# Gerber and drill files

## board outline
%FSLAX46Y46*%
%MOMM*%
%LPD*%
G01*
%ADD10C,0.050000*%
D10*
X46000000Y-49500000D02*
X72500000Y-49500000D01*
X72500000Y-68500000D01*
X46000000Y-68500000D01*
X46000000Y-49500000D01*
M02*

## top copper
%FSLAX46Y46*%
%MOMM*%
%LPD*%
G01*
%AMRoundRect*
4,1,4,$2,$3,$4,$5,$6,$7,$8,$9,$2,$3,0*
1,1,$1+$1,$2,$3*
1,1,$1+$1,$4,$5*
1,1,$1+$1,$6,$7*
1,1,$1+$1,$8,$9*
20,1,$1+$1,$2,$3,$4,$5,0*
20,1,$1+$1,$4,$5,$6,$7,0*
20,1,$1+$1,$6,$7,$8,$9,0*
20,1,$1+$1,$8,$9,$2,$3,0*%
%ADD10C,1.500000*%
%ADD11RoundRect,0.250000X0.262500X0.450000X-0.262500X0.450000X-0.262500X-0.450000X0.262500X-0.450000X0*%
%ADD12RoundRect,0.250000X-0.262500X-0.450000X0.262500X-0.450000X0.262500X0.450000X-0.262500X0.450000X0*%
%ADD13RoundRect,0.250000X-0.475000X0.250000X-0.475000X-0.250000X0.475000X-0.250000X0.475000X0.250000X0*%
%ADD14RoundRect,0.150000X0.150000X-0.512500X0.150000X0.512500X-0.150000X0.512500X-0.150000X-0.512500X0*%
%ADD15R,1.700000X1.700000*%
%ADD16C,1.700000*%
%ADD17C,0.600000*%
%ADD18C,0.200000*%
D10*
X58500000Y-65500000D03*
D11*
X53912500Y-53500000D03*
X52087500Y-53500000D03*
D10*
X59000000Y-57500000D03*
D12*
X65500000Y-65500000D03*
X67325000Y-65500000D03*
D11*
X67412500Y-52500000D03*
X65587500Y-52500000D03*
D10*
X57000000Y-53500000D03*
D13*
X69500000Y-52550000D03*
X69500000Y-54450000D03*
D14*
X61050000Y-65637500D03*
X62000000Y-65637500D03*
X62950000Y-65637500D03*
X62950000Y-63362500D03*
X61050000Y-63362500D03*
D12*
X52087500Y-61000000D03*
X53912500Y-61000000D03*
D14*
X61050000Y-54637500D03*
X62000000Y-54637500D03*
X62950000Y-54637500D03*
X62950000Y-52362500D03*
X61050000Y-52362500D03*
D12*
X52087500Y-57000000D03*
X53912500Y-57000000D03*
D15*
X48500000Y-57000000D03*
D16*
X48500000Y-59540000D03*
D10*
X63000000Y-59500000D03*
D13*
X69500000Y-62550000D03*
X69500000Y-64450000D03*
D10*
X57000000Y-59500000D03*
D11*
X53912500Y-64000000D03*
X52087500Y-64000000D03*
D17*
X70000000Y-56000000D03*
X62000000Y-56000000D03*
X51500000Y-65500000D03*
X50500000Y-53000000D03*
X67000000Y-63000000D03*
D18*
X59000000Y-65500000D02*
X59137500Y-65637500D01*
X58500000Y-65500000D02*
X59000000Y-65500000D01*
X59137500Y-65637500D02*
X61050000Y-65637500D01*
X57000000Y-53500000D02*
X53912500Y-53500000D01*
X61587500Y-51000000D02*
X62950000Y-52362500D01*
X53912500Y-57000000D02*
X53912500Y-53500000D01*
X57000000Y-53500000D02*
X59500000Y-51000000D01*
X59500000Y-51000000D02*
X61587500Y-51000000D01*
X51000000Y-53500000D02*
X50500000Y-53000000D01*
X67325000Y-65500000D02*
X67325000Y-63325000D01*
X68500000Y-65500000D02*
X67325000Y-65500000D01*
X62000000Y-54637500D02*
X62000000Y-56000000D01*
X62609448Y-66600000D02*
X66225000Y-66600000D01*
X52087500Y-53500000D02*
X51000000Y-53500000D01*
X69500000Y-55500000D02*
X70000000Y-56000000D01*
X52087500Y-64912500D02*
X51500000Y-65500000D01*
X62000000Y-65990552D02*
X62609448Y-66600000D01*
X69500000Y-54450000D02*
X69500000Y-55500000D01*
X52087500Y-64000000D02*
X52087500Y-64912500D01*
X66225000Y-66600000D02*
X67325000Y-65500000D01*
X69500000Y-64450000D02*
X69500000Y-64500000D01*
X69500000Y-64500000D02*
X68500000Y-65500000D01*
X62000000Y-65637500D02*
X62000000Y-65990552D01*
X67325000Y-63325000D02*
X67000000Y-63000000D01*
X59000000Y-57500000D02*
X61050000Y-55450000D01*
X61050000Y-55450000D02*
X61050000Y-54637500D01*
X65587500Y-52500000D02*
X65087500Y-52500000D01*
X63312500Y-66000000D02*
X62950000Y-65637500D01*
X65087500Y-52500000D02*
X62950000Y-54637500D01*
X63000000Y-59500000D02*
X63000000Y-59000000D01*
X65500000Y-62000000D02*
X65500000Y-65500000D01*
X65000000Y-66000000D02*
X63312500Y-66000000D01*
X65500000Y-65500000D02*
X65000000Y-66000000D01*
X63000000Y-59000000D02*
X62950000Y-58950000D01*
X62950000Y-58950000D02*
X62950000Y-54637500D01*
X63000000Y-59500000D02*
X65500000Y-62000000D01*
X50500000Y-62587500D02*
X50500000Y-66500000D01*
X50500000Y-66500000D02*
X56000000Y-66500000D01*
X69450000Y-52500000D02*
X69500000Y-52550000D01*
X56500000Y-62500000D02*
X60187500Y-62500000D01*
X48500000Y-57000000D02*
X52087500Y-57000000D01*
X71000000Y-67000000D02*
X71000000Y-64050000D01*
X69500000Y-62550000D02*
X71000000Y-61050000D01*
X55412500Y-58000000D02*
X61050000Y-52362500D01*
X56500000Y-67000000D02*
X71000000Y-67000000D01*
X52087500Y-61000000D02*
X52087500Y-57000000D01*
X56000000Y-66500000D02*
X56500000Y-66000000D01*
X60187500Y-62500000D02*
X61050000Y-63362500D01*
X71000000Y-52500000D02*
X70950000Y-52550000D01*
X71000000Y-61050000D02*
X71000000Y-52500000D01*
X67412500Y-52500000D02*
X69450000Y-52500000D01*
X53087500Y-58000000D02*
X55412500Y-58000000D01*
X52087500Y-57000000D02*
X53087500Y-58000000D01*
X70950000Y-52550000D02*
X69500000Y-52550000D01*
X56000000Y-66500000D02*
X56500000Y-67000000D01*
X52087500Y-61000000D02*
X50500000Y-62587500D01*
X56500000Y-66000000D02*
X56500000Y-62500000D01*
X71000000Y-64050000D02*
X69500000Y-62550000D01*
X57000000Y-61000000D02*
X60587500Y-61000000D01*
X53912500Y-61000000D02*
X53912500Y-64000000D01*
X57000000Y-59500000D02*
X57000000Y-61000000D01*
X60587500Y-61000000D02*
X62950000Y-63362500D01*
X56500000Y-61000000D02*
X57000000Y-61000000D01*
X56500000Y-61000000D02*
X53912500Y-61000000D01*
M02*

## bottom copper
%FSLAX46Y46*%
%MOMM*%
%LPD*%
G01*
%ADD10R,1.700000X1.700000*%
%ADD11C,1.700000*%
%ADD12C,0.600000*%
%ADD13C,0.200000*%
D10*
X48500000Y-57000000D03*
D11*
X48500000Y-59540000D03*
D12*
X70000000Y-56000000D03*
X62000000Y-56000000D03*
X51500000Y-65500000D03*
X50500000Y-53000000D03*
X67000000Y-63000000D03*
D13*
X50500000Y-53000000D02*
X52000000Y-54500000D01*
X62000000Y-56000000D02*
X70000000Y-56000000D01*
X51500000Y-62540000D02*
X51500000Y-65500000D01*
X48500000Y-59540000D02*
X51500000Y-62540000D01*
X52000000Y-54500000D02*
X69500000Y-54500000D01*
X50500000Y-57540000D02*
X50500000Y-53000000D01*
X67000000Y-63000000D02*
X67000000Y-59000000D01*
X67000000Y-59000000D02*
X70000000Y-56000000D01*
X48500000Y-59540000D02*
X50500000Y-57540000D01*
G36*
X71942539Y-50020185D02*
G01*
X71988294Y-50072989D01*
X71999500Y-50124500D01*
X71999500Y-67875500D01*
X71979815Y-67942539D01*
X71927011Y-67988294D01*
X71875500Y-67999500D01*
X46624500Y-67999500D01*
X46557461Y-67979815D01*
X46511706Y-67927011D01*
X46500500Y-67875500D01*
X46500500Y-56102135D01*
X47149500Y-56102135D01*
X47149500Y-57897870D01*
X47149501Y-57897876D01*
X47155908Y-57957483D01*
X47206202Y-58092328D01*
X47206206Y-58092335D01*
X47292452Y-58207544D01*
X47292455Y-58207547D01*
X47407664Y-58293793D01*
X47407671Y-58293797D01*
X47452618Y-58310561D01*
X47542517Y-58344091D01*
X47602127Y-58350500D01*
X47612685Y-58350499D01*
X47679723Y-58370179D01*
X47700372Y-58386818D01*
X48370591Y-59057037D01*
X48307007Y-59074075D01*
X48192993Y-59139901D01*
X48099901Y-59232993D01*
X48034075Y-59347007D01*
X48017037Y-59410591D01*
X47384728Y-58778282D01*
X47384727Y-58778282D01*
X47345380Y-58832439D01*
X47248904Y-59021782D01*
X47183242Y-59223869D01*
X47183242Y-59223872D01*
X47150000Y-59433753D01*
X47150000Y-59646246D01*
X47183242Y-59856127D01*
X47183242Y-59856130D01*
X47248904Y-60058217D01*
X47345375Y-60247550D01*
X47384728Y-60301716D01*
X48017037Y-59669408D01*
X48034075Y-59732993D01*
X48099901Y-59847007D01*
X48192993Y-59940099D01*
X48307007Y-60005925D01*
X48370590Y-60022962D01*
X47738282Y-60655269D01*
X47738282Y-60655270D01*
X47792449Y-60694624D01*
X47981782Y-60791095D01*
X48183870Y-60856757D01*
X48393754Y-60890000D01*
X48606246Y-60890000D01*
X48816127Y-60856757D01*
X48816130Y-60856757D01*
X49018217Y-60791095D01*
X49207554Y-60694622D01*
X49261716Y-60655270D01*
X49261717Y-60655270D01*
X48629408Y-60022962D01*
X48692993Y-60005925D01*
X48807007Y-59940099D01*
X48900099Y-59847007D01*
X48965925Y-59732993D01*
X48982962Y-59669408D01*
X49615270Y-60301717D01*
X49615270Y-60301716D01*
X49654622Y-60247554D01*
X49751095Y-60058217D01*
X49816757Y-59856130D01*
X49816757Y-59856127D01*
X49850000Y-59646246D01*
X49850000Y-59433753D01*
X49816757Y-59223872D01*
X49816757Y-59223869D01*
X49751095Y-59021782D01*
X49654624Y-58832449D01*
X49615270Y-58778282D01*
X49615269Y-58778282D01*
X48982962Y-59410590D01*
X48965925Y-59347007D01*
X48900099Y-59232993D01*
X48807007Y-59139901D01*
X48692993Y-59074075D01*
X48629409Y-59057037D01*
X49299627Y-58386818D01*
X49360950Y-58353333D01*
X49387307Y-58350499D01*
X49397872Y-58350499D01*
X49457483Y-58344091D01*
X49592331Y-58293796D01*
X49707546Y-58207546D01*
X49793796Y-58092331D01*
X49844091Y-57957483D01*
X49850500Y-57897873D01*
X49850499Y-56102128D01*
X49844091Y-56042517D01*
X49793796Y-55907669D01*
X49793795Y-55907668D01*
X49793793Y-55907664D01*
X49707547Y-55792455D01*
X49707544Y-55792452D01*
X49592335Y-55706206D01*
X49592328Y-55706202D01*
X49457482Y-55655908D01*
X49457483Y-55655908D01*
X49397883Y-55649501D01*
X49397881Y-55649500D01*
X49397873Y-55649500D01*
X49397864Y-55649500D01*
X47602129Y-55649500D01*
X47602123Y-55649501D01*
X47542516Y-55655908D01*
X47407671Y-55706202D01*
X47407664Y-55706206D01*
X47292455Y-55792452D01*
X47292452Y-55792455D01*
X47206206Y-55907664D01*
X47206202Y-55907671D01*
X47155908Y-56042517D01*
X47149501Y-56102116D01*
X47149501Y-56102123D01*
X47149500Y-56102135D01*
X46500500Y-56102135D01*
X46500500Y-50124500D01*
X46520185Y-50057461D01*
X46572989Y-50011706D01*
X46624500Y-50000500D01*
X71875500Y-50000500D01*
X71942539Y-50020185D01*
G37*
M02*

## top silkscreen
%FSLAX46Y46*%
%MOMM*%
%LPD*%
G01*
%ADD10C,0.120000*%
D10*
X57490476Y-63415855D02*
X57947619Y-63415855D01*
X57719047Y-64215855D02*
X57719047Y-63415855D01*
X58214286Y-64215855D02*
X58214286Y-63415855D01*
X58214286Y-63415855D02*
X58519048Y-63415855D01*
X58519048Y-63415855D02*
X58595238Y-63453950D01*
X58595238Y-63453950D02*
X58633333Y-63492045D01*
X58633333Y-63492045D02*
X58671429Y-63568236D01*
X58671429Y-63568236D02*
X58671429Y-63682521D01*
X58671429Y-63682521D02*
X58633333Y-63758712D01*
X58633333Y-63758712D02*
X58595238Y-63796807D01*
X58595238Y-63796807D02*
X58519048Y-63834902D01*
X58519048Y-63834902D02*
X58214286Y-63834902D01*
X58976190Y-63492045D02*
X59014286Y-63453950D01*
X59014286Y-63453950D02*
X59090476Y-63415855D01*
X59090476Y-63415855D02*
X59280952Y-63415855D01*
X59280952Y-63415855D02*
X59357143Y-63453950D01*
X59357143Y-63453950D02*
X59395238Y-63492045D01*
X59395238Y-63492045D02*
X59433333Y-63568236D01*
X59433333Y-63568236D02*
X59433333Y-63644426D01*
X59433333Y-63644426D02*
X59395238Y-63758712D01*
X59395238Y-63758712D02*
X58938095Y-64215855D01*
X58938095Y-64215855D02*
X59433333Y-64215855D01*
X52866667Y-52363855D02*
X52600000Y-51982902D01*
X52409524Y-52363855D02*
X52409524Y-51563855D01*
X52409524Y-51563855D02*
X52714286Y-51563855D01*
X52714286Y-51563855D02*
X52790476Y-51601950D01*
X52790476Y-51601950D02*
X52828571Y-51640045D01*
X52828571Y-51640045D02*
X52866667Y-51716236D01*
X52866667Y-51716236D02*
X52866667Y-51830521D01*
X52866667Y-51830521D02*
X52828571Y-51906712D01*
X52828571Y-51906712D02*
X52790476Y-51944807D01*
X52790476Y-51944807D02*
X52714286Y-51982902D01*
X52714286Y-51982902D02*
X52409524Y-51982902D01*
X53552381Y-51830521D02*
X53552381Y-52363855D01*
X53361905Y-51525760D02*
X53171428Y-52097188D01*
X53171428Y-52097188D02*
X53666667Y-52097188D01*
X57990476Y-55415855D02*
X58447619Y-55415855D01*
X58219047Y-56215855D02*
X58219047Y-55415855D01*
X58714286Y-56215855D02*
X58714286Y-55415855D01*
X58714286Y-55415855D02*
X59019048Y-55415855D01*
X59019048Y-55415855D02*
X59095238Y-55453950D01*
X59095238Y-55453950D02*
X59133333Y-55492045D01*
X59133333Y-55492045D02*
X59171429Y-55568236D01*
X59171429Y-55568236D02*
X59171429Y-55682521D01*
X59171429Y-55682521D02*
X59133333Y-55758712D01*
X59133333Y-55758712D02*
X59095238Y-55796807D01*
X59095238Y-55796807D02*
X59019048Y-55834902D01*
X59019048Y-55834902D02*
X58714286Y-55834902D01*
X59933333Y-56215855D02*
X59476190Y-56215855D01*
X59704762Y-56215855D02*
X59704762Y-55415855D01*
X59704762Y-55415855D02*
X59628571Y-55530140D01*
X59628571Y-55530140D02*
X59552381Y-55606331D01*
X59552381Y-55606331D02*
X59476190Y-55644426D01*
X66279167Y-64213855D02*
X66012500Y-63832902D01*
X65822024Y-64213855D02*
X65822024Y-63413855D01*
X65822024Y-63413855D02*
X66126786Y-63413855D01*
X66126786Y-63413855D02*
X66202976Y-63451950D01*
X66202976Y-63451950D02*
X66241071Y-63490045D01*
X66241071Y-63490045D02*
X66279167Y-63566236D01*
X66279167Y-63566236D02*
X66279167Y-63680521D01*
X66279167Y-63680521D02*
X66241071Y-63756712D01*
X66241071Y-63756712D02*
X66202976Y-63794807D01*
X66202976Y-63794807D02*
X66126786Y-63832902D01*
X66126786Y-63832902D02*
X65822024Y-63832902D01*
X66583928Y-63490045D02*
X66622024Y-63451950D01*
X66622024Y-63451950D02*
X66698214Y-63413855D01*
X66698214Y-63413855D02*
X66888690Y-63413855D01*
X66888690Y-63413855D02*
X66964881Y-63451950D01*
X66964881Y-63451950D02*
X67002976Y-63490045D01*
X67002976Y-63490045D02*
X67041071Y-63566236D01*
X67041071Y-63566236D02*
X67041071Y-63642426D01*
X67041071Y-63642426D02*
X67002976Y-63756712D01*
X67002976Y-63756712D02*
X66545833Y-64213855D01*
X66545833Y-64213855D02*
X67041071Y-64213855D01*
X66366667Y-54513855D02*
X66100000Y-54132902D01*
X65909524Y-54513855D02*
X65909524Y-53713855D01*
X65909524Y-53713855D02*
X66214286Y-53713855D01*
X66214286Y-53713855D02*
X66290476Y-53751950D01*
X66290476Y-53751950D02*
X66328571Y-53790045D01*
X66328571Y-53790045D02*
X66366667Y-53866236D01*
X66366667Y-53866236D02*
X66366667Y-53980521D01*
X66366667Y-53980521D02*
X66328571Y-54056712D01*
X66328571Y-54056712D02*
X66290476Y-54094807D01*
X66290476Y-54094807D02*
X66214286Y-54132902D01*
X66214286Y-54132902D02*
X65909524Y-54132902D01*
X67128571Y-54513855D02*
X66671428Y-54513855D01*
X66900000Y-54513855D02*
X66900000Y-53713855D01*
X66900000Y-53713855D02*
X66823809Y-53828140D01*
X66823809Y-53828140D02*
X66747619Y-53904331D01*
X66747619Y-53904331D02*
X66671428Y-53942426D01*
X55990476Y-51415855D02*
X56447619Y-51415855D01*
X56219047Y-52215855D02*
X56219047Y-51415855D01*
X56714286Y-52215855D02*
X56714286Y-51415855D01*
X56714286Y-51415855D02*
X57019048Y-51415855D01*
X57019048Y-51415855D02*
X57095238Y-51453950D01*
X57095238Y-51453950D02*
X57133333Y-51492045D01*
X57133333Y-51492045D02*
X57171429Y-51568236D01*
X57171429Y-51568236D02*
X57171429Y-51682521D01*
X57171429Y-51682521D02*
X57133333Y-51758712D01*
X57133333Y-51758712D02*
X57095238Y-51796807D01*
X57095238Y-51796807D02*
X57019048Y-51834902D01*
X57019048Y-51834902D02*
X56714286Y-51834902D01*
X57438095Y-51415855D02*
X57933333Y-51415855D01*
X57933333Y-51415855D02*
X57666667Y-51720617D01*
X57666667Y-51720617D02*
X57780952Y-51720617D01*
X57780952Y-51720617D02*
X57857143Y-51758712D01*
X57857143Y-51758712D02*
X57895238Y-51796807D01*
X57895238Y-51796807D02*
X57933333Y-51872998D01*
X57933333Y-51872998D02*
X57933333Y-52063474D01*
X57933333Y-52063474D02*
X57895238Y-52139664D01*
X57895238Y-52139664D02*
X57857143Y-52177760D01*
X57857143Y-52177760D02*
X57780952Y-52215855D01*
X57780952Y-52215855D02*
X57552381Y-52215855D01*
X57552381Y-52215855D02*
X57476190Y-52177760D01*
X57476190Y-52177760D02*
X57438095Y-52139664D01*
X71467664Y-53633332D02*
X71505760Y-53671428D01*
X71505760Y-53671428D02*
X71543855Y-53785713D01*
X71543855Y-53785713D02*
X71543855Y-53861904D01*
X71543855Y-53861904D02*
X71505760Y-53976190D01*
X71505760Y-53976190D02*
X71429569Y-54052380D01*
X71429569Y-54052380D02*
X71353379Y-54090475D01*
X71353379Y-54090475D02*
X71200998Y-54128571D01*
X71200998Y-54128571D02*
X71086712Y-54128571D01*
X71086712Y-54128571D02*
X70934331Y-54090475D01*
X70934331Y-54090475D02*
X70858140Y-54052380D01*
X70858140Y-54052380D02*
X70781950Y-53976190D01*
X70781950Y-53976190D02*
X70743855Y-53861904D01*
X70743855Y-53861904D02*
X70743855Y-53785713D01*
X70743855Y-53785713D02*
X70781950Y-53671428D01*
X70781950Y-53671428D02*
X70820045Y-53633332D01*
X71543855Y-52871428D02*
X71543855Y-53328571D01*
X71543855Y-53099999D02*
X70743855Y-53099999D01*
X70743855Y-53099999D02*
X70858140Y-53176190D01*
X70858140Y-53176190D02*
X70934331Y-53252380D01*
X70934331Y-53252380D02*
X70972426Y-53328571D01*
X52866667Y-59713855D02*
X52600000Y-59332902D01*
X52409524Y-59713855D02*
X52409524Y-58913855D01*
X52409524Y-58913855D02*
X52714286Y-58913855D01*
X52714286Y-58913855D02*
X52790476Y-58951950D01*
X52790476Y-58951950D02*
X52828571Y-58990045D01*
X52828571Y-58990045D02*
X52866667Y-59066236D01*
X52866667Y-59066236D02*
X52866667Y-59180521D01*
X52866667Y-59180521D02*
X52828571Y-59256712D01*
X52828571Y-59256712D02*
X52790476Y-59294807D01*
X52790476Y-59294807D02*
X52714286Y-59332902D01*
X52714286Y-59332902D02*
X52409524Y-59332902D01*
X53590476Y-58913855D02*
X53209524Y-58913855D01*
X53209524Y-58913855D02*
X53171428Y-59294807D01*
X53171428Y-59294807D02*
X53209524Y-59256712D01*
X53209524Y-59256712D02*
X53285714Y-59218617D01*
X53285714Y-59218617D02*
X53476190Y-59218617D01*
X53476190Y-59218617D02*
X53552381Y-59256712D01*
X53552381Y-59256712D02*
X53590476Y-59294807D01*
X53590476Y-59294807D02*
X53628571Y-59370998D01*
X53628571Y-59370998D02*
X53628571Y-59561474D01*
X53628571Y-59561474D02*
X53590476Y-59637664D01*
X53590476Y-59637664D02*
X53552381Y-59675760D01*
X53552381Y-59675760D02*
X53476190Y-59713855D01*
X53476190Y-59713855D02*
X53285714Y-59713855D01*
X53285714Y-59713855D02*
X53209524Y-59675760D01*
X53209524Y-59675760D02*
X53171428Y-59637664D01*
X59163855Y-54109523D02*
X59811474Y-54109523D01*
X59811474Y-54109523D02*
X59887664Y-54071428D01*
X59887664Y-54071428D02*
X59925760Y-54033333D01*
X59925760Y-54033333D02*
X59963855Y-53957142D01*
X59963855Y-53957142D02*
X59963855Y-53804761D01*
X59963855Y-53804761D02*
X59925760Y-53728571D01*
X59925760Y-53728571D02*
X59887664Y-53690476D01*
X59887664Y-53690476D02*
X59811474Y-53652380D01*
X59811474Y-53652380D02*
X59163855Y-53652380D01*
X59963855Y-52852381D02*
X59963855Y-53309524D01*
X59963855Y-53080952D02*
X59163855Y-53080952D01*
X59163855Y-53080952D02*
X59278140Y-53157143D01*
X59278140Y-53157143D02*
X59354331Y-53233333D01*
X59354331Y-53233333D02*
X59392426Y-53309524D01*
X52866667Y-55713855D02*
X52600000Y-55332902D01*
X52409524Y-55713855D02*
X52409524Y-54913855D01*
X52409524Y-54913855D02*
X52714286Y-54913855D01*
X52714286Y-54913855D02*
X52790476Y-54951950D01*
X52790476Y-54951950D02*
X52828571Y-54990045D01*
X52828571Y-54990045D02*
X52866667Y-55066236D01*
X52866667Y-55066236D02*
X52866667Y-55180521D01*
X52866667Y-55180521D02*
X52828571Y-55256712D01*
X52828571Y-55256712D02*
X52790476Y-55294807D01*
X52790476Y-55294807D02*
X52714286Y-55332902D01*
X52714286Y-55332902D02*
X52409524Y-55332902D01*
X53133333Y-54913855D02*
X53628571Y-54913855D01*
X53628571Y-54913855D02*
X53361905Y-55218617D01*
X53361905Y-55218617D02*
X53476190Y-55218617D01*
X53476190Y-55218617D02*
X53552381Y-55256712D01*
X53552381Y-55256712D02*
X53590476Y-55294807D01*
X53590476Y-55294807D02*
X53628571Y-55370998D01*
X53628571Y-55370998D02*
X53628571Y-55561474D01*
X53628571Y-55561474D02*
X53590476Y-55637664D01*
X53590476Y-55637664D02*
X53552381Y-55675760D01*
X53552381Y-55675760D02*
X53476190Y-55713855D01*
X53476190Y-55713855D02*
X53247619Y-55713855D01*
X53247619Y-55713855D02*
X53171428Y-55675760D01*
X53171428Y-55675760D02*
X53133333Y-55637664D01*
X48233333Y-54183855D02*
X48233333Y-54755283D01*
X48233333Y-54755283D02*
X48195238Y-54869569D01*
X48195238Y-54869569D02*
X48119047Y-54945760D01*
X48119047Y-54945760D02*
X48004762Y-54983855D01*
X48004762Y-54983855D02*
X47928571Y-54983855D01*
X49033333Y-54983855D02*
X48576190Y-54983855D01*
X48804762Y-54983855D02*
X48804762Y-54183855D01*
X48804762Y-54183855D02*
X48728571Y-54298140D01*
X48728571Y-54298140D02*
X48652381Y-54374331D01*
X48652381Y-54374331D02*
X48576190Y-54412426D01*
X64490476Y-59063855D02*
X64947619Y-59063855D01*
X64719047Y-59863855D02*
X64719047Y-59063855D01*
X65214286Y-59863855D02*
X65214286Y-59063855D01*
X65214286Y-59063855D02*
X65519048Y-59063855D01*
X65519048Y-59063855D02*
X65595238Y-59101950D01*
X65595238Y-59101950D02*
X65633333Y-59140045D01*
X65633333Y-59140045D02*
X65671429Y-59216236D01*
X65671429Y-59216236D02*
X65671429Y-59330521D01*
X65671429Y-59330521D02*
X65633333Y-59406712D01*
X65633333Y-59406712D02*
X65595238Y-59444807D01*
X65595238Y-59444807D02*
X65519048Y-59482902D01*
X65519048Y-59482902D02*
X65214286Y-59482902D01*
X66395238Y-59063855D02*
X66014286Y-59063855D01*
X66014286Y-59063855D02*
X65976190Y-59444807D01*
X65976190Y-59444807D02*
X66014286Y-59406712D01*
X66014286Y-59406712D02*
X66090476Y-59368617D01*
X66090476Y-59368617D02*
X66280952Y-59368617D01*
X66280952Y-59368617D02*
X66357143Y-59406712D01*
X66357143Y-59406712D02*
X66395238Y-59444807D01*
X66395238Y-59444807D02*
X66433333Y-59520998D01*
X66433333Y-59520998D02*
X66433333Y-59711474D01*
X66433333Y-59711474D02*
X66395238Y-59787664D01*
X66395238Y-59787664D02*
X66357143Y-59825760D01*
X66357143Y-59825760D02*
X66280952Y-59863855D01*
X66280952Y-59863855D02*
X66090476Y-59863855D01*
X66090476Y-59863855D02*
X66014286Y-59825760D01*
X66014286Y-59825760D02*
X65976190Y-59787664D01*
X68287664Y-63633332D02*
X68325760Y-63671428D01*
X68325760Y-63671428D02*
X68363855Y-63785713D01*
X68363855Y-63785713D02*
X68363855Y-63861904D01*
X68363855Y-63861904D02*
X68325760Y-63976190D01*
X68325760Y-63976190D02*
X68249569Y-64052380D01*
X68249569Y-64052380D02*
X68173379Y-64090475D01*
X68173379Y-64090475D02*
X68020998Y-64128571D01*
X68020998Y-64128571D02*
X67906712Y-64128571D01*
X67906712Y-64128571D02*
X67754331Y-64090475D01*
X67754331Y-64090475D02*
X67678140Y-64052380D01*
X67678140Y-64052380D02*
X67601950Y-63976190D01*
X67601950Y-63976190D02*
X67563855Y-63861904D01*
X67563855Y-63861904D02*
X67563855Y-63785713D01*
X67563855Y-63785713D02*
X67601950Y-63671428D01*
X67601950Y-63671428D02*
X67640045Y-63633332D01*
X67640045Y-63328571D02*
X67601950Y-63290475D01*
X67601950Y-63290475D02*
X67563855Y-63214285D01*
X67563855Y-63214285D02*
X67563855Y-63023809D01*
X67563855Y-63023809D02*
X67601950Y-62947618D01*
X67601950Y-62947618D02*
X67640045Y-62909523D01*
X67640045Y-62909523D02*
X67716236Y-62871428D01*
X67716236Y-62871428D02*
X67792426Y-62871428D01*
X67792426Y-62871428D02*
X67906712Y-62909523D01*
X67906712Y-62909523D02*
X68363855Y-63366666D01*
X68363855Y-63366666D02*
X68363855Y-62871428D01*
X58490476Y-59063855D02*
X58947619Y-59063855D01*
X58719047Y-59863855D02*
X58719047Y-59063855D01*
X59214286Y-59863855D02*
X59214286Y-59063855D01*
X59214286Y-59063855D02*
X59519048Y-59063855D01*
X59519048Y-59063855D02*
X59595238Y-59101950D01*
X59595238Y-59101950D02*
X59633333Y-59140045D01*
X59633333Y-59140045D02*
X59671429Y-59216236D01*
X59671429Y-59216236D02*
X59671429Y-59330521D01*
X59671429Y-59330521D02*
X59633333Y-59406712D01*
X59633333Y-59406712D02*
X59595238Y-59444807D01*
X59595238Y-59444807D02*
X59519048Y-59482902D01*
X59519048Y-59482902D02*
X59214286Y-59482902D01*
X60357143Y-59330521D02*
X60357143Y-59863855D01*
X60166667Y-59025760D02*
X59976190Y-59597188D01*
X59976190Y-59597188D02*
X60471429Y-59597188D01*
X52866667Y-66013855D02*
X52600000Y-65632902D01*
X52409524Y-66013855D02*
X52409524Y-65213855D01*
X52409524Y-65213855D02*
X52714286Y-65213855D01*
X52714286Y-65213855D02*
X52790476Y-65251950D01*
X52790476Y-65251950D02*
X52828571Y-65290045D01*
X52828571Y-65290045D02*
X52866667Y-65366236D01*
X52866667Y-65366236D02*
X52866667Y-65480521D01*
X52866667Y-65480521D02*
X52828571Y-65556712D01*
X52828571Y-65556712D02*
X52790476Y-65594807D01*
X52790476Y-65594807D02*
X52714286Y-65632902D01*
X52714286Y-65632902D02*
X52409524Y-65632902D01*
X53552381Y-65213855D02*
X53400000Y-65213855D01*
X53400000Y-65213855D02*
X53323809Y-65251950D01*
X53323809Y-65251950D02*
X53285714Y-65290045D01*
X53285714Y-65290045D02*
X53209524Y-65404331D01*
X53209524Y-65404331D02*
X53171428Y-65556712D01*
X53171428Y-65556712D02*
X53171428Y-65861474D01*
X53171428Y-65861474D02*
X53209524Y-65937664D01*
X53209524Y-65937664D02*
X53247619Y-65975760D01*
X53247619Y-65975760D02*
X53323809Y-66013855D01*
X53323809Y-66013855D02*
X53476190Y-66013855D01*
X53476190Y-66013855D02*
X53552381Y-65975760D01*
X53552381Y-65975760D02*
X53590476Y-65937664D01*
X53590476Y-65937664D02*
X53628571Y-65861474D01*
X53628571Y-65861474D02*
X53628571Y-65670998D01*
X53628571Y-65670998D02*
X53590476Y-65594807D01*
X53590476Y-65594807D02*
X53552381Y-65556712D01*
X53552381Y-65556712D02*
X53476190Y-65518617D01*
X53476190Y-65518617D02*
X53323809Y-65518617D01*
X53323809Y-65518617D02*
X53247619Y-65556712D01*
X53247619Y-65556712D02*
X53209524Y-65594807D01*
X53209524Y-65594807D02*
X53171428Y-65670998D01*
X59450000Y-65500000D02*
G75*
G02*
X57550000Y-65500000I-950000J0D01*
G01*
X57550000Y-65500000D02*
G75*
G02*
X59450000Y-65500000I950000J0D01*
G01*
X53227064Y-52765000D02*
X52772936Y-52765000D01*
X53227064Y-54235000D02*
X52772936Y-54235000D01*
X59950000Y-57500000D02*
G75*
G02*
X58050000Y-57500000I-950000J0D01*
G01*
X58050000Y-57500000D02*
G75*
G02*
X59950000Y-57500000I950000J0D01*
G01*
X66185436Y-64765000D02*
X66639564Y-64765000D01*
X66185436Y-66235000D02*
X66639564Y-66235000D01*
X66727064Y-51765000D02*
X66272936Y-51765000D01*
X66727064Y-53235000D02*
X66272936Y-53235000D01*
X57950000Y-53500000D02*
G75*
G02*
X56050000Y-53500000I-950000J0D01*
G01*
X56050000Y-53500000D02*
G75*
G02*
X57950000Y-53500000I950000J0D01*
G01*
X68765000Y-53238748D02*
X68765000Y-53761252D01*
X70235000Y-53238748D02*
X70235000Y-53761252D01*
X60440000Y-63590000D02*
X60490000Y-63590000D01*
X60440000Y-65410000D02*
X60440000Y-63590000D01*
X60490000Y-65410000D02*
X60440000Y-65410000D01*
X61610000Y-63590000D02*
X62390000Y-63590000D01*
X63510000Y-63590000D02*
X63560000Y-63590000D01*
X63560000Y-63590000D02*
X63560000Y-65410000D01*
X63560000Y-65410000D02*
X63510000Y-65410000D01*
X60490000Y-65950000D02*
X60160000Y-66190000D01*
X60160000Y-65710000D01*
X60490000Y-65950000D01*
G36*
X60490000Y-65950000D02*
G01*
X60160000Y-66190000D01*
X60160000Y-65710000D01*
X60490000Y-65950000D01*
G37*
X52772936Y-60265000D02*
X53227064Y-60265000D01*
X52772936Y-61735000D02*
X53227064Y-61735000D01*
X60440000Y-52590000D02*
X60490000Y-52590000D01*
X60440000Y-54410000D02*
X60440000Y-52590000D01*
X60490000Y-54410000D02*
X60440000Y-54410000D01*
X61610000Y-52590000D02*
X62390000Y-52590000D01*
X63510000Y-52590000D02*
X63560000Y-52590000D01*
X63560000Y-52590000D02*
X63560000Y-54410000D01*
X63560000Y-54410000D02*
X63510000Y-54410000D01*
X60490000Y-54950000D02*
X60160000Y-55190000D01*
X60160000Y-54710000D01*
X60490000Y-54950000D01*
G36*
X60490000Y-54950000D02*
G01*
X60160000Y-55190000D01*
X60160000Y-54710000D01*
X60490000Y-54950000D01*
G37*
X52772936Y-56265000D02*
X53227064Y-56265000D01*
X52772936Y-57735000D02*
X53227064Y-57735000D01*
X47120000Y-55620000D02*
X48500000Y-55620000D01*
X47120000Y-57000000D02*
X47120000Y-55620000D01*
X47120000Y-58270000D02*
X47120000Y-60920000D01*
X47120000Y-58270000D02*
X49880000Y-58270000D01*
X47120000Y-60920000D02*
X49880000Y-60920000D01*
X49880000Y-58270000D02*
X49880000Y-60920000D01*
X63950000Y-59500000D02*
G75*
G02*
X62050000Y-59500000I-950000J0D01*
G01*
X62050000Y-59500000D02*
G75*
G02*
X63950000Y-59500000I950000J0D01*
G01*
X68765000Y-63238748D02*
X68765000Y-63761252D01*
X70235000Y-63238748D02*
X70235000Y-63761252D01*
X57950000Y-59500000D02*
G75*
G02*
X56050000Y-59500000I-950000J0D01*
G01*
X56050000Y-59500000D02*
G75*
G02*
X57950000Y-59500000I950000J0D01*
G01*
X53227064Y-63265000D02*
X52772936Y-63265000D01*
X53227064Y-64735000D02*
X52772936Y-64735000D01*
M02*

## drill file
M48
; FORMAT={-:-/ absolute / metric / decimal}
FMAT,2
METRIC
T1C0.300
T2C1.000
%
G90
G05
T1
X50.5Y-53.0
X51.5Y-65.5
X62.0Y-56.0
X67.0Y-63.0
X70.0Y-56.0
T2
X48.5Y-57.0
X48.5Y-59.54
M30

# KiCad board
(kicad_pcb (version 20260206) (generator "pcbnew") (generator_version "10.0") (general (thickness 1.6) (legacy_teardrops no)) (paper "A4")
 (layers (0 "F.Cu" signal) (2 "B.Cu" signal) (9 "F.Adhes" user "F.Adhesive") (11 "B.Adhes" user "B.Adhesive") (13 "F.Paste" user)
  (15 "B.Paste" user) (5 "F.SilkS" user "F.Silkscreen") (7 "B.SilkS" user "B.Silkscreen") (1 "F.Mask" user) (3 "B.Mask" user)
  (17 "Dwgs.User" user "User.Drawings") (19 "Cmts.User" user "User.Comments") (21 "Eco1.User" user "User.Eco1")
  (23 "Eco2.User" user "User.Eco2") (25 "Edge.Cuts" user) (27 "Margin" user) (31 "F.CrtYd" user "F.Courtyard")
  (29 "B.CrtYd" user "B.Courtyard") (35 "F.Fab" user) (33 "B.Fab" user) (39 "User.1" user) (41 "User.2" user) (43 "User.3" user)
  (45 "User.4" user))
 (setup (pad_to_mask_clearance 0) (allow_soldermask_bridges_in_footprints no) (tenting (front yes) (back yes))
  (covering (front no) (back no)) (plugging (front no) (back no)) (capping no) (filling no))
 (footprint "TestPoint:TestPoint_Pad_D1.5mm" (layer "F.Cu") (at 58.5 65.5)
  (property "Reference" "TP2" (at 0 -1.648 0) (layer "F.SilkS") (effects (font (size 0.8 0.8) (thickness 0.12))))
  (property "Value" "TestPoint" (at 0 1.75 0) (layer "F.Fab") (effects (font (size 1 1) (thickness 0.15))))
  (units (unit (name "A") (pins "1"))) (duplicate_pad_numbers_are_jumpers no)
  (fp_circle (center 0 0) (end 0 0.95) (stroke (width 0.12) (type solid)) (fill no) (layer "F.SilkS"))
  (pad "1" smd circle (at 0 0) (size 1.5 1.5) (layers "F.Cu" "F.Mask") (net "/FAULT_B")))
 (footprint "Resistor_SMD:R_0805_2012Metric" (layer "F.Cu") (at 53 53.5 180)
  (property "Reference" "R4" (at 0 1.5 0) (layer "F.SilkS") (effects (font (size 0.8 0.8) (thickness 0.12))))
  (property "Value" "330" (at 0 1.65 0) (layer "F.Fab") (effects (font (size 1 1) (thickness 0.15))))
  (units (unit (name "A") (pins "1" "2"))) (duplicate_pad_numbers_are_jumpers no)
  (fp_line (start -0.227064 0.735) (end 0.227064 0.735) (stroke (width 0.12) (type solid)) (layer "F.SilkS"))
  (fp_line (start -0.227064 -0.735) (end 0.227064 -0.735) (stroke (width 0.12) (type solid)) (layer "F.SilkS"))
  (pad "1" smd roundrect (at -0.9125 0 180) (size 1.025 1.4) (layers "F.Cu" "F.Mask" "F.Paste") (roundrect_rratio 0.243902) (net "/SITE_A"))
  (pad "2" smd roundrect (at 0.9125 0 180) (size 1.025 1.4) (layers "F.Cu" "F.Mask" "F.Paste") (roundrect_rratio 0.243902) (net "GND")))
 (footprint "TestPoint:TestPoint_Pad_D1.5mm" (layer "F.Cu") (at 59 57.5)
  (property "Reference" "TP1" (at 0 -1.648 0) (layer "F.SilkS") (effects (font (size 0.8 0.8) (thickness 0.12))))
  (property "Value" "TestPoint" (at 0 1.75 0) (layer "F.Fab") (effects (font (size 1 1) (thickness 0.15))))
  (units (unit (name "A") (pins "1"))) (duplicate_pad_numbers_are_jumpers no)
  (fp_circle (center 0 0) (end 0 0.95) (stroke (width 0.12) (type solid)) (fill no) (layer "F.SilkS"))
  (pad "1" smd circle (at 0 0) (size 1.5 1.5) (layers "F.Cu" "F.Mask") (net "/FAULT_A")))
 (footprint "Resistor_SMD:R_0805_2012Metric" (layer "F.Cu") (at 66.4125 65.5)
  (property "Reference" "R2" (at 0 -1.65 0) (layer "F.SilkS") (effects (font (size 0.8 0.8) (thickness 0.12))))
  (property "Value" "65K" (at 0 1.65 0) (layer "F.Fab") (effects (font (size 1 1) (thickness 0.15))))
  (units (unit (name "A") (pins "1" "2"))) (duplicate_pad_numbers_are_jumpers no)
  (fp_line (start -0.227064 -0.735) (end 0.227064 -0.735) (stroke (width 0.12) (type solid)) (layer "F.SilkS"))
  (fp_line (start -0.227064 0.735) (end 0.227064 0.735) (stroke (width 0.12) (type solid)) (layer "F.SilkS"))
  (pad "1" smd roundrect (at -0.9125 0) (size 1.025 1.4) (layers "F.Cu" "F.Mask" "F.Paste") (roundrect_rratio 0.243902) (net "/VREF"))
  (pad "2" smd roundrect (at 0.9125 0) (size 1.025 1.4) (layers "F.Cu" "F.Mask" "F.Paste") (roundrect_rratio 0.243902) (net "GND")))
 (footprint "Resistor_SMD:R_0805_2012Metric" (layer "F.Cu") (at 66.5 52.5 180)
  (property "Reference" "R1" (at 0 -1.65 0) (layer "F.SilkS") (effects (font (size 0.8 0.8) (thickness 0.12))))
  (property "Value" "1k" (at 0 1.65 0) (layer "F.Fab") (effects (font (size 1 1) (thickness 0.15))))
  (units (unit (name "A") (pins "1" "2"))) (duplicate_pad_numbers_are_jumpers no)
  (fp_line (start -0.227064 0.735) (end 0.227064 0.735) (stroke (width 0.12) (type solid)) (layer "F.SilkS"))
  (fp_line (start -0.227064 -0.735) (end 0.227064 -0.735) (stroke (width 0.12) (type solid)) (layer "F.SilkS"))
  (pad "1" smd roundrect (at -0.9125 0 180) (size 1.025 1.4) (layers "F.Cu" "F.Mask" "F.Paste") (roundrect_rratio 0.243902) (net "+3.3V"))
  (pad "2" smd roundrect (at 0.9125 0 180) (size 1.025 1.4) (layers "F.Cu" "F.Mask" "F.Paste") (roundrect_rratio 0.243902) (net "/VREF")))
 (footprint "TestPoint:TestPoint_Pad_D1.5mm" (layer "F.Cu") (at 57 53.5)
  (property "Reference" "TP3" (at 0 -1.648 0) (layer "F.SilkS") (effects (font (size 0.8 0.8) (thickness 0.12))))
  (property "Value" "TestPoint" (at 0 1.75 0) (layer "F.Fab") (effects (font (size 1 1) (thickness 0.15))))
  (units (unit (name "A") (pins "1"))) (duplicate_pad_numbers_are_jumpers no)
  (fp_circle (center 0 0) (end 0 0.95) (stroke (width 0.12) (type solid)) (fill no) (layer "F.SilkS"))
  (pad "1" smd circle (at 0 0) (size 1.5 1.5) (layers "F.Cu" "F.Mask") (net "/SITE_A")))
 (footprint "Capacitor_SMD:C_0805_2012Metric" (layer "F.Cu") (at 69.5 53.5 -90)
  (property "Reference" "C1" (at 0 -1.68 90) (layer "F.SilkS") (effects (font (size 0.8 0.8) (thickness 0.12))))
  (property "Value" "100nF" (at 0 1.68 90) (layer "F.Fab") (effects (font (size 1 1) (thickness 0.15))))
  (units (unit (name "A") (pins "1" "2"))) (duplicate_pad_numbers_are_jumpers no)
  (fp_line (start -0.261252 0.735) (end 0.261252 0.735) (stroke (width 0.12) (type solid)) (layer "F.SilkS"))
  (fp_line (start -0.261252 -0.735) (end 0.261252 -0.735) (stroke (width 0.12) (type solid)) (layer "F.SilkS"))
  (pad "1" smd roundrect (at -0.95 0 270) (size 1 1.45) (layers "F.Cu" "F.Mask" "F.Paste") (roundrect_rratio 0.25) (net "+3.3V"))
  (pad "2" smd roundrect (at 0.95 0 270) (size 1 1.45) (layers "F.Cu" "F.Mask" "F.Paste") (roundrect_rratio 0.25) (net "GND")))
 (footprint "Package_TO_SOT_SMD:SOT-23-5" (layer "F.Cu") (at 62 64.5 90)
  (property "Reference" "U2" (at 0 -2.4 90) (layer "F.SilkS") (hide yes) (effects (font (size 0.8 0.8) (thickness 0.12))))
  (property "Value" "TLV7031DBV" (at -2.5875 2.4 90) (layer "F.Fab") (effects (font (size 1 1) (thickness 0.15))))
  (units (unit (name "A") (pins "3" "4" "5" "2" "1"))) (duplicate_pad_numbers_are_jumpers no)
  (fp_line (start 0.91 -1.56) (end 0.91 -1.51) (stroke (width 0.12) (type solid)) (layer "F.SilkS"))
  (fp_line (start -0.91 -1.56) (end 0.91 -1.56) (stroke (width 0.12) (type solid)) (layer "F.SilkS"))
  (fp_line (start -0.91 -1.51) (end -0.91 -1.56) (stroke (width 0.12) (type solid)) (layer "F.SilkS"))
  (fp_line (start 0.91 -0.39) (end 0.91 0.39) (stroke (width 0.12) (type solid)) (layer "F.SilkS"))
  (fp_line (start 0.91 1.51) (end 0.91 1.56) (stroke (width 0.12) (type solid)) (layer "F.SilkS"))
  (fp_line (start 0.91 1.56) (end -0.91 1.56) (stroke (width 0.12) (type solid)) (layer "F.SilkS"))
  (fp_line (start -0.91 1.56) (end -0.91 1.51) (stroke (width 0.12) (type solid)) (layer "F.SilkS"))
  (fp_poly (pts (xy -1.45 -1.51) (xy -1.69 -1.84) (xy -1.21 -1.84)) (stroke (width 0.12) (type solid)) (fill yes) (layer "F.SilkS"))
  (pad "1" smd roundrect (at -1.1375 -0.95 90) (size 1.325 0.6) (layers "F.Cu" "F.Mask" "F.Paste") (roundrect_rratio 0.25) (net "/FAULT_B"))
  (pad "2" smd roundrect (at -1.1375 0 90) (size 1.325 0.6) (layers "F.Cu" "F.Mask" "F.Paste") (roundrect_rratio 0.25) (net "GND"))
  (pad "3" smd roundrect (at -1.1375 0.95 90) (size 1.325 0.6) (layers "F.Cu" "F.Mask" "F.Paste") (roundrect_rratio 0.25) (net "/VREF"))
  (pad "4" smd roundrect (at 1.1375 0.95 90) (size 1.325 0.6) (layers "F.Cu" "F.Mask" "F.Paste") (roundrect_rratio 0.25) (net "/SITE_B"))
  (pad "5" smd roundrect (at 1.1375 -0.95 90) (size 1.325 0.6) (layers "F.Cu" "F.Mask" "F.Paste") (roundrect_rratio 0.25) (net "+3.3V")))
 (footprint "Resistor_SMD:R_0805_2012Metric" (layer "F.Cu") (at 53 61)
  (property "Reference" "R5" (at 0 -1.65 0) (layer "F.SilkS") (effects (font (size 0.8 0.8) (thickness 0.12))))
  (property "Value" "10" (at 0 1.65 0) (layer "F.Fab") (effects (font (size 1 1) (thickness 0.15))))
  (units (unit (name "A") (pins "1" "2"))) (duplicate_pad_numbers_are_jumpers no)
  (fp_line (start -0.227064 -0.735) (end 0.227064 -0.735) (stroke (width 0.12) (type solid)) (layer "F.SilkS"))
  (fp_line (start -0.227064 0.735) (end 0.227064 0.735) (stroke (width 0.12) (type solid)) (layer "F.SilkS"))
  (pad "1" smd roundrect (at -0.9125 0) (size 1.025 1.4) (layers "F.Cu" "F.Mask" "F.Paste") (roundrect_rratio 0.243902) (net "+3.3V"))
  (pad "2" smd roundrect (at 0.9125 0) (size 1.025 1.4) (layers "F.Cu" "F.Mask" "F.Paste") (roundrect_rratio 0.243902) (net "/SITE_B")))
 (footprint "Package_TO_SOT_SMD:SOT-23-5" (layer "F.Cu") (at 62 53.5 90)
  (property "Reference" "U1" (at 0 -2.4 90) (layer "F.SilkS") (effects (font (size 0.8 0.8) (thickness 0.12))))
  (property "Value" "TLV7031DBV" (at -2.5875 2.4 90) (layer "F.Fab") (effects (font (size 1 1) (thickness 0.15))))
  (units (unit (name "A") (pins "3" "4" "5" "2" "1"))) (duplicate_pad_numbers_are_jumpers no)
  (fp_line (start 0.91 -1.56) (end 0.91 -1.51) (stroke (width 0.12) (type solid)) (layer "F.SilkS"))
  (fp_line (start -0.91 -1.56) (end 0.91 -1.56) (stroke (width 0.12) (type solid)) (layer "F.SilkS"))
  (fp_line (start -0.91 -1.51) (end -0.91 -1.56) (stroke (width 0.12) (type solid)) (layer "F.SilkS"))
  (fp_line (start 0.91 -0.39) (end 0.91 0.39) (stroke (width 0.12) (type solid)) (layer "F.SilkS"))
  (fp_line (start 0.91 1.51) (end 0.91 1.56) (stroke (width 0.12) (type solid)) (layer "F.SilkS"))
  (fp_line (start 0.91 1.56) (end -0.91 1.56) (stroke (width 0.12) (type solid)) (layer "F.SilkS"))
  (fp_line (start -0.91 1.56) (end -0.91 1.51) (stroke (width 0.12) (type solid)) (layer "F.SilkS"))
  (fp_poly (pts (xy -1.45 -1.51) (xy -1.69 -1.84) (xy -1.21 -1.84)) (stroke (width 0.12) (type solid)) (fill yes) (layer "F.SilkS"))
  (pad "1" smd roundrect (at -1.1375 -0.95 90) (size 1.325 0.6) (layers "F.Cu" "F.Mask" "F.Paste") (roundrect_rratio 0.25) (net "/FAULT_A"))
  (pad "2" smd roundrect (at -1.1375 0 90) (size 1.325 0.6) (layers "F.Cu" "F.Mask" "F.Paste") (roundrect_rratio 0.25) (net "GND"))
  (pad "3" smd roundrect (at -1.1375 0.95 90) (size 1.325 0.6) (layers "F.Cu" "F.Mask" "F.Paste") (roundrect_rratio 0.25) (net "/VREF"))
  (pad "4" smd roundrect (at 1.1375 0.95 90) (size 1.325 0.6) (layers "F.Cu" "F.Mask" "F.Paste") (roundrect_rratio 0.25) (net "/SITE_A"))
  (pad "5" smd roundrect (at 1.1375 -0.95 90) (size 1.325 0.6) (layers "F.Cu" "F.Mask" "F.Paste") (roundrect_rratio 0.25) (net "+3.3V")))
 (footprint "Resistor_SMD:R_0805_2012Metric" (layer "F.Cu") (at 53 57)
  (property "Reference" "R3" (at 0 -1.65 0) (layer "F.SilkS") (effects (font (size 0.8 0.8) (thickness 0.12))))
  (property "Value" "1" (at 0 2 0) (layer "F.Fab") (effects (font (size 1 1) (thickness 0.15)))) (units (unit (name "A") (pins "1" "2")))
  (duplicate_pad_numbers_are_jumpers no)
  (fp_line (start -0.227064 -0.735) (end 0.227064 -0.735) (stroke (width 0.12) (type solid)) (layer "F.SilkS"))
  (fp_line (start -0.227064 0.735) (end 0.227064 0.735) (stroke (width 0.12) (type solid)) (layer "F.SilkS"))
  (pad "1" smd roundrect (at -0.9125 0) (size 1.025 1.4) (layers "F.Cu" "F.Mask" "F.Paste") (roundrect_rratio 0.243902) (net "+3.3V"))
  (pad "2" smd roundrect (at 0.9125 0) (size 1.025 1.4) (layers "F.Cu" "F.Mask" "F.Paste") (roundrect_rratio 0.243902) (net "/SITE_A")))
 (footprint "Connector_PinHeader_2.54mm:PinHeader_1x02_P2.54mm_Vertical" (layer "F.Cu") (at 48.5 57)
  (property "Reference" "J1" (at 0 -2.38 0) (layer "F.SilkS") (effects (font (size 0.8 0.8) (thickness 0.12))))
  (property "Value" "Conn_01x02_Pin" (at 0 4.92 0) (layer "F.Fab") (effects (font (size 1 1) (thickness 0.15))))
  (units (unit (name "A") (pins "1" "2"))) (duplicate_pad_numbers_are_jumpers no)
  (fp_line (start -1.38 -1.38) (end 0 -1.38) (stroke (width 0.12) (type solid)) (layer "F.SilkS"))
  (fp_line (start -1.38 0) (end -1.38 -1.38) (stroke (width 0.12) (type solid)) (layer "F.SilkS"))
  (fp_line (start -1.38 1.27) (end -1.38 3.92) (stroke (width 0.12) (type solid)) (layer "F.SilkS"))
  (fp_line (start -1.38 1.27) (end 1.38 1.27) (stroke (width 0.12) (type solid)) (layer "F.SilkS"))
  (fp_line (start -1.38 3.92) (end 1.38 3.92) (stroke (width 0.12) (type solid)) (layer "F.SilkS"))
  (fp_line (start 1.38 1.27) (end 1.38 3.92) (stroke (width 0.12) (type solid)) (layer "F.SilkS"))
  (pad "1" thru_hole rect (at 0 0) (size 1.7 1.7) (drill 1) (layers "*.Cu" "*.Mask") (remove_unused_layers no) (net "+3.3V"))
  (pad "2" thru_hole circle (at 0 2.54) (size 1.7 1.7) (drill 1) (layers "*.Cu" "*.Mask") (remove_unused_layers no) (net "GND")))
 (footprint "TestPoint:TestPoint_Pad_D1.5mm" (layer "F.Cu") (at 63 59.5)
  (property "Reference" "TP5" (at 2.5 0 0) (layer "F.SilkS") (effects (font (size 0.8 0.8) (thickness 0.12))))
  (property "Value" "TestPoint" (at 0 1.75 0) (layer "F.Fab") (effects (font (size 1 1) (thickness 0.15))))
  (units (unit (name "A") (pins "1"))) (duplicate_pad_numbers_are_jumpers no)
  (fp_circle (center 0 0) (end 0 0.95) (stroke (width 0.12) (type solid)) (fill no) (layer "F.SilkS"))
  (pad "1" smd circle (at 0 0) (size 1.5 1.5) (layers "F.Cu" "F.Mask") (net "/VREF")))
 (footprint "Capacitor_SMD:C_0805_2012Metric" (layer "F.Cu") (at 69.5 63.5 -90)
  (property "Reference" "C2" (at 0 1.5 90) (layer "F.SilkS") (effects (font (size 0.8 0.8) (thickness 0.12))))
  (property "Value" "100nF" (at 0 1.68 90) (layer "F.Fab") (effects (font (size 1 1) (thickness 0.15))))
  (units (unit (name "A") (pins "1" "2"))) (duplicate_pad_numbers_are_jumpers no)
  (fp_line (start -0.261252 0.735) (end 0.261252 0.735) (stroke (width 0.12) (type solid)) (layer "F.SilkS"))
  (fp_line (start -0.261252 -0.735) (end 0.261252 -0.735) (stroke (width 0.12) (type solid)) (layer "F.SilkS"))
  (pad "1" smd roundrect (at -0.95 0 270) (size 1 1.45) (layers "F.Cu" "F.Mask" "F.Paste") (roundrect_rratio 0.25) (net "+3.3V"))
  (pad "2" smd roundrect (at 0.95 0 270) (size 1 1.45) (layers "F.Cu" "F.Mask" "F.Paste") (roundrect_rratio 0.25) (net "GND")))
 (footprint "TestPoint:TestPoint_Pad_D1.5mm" (layer "F.Cu") (at 57 59.5)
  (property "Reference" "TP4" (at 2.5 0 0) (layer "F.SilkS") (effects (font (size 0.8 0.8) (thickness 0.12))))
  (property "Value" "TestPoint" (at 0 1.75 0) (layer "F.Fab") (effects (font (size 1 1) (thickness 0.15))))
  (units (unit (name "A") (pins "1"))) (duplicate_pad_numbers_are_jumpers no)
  (fp_circle (center 0 0) (end 0 0.95) (stroke (width 0.12) (type solid)) (fill no) (layer "F.SilkS"))
  (pad "1" smd circle (at 0 0) (size 1.5 1.5) (layers "F.Cu" "F.Mask") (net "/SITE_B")))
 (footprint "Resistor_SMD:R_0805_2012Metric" (layer "F.Cu") (at 53 64 180)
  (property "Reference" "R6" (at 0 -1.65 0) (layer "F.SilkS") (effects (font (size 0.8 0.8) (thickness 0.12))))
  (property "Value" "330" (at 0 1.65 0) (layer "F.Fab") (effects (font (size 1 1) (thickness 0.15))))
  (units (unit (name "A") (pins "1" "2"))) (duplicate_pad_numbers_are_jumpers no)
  (fp_line (start -0.227064 0.735) (end 0.227064 0.735) (stroke (width 0.12) (type solid)) (layer "F.SilkS"))
  (fp_line (start -0.227064 -0.735) (end 0.227064 -0.735) (stroke (width 0.12) (type solid)) (layer "F.SilkS"))
  (pad "1" smd roundrect (at -0.9125 0 180) (size 1.025 1.4) (layers "F.Cu" "F.Mask" "F.Paste") (roundrect_rratio 0.243902) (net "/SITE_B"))
  (pad "2" smd roundrect (at 0.9125 0 180) (size 1.025 1.4) (layers "F.Cu" "F.Mask" "F.Paste") (roundrect_rratio 0.243902) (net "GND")))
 (gr_rect (start 46 49.5) (end 72.5 68.5) (stroke (width 0.05) (type default)) (fill no) (layer "Edge.Cuts"))
 (segment (start 59 65.5) (end 59.1375 65.6375) (width 0.2) (layer "F.Cu") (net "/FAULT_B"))
 (segment (start 58.5 65.5) (end 59 65.5) (width 0.2) (layer "F.Cu") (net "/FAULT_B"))
 (segment (start 59.1375 65.6375) (end 61.05 65.6375) (width 0.2) (layer "F.Cu") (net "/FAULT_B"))
 (segment (start 57 53.5) (end 53.9125 53.5) (width 0.2) (layer "F.Cu") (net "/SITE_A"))
 (segment (start 61.5875 51) (end 62.95 52.3625) (width 0.2) (layer "F.Cu") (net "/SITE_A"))
 (segment (start 53.9125 57) (end 53.9125 53.5) (width 0.2) (layer "F.Cu") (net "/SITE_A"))
 (segment (start 57 53.5) (end 59.5 51) (width 0.2) (layer "F.Cu") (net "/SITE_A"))
 (segment (start 59.5 51) (end 61.5875 51) (width 0.2) (layer "F.Cu") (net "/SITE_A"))
 (segment (start 51 53.5) (end 50.5 53) (width 0.2) (layer "F.Cu") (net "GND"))
 (segment (start 67.325 65.5) (end 67.325 63.325) (width 0.2) (layer "F.Cu") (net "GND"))
 (segment (start 68.5 65.5) (end 67.325 65.5) (width 0.2) (layer "F.Cu") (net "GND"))
 (segment (start 62 54.6375) (end 62 56) (width 0.2) (layer "F.Cu") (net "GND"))
 (segment (start 62.609448 66.6) (end 66.225 66.6) (width 0.2) (layer "F.Cu") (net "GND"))
 (segment (start 52.0875 53.5) (end 51 53.5) (width 0.2) (layer "F.Cu") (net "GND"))
 (segment (start 69.5 55.5) (end 70 56) (width 0.2) (layer "F.Cu") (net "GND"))
 (segment (start 52.0875 64.9125) (end 51.5 65.5) (width 0.2) (layer "F.Cu") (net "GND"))
 (segment (start 62 65.990552) (end 62.609448 66.6) (width 0.2) (layer "F.Cu") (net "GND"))
 (segment (start 69.5 54.45) (end 69.5 55.5) (width 0.2) (layer "F.Cu") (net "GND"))
 (segment (start 52.0875 64) (end 52.0875 64.9125) (width 0.2) (layer "F.Cu") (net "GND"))
 (segment (start 66.225 66.6) (end 67.325 65.5) (width 0.2) (layer "F.Cu") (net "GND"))
 (segment (start 69.5 64.45) (end 69.5 64.5) (width 0.2) (layer "F.Cu") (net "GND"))
 (segment (start 69.5 64.5) (end 68.5 65.5) (width 0.2) (layer "F.Cu") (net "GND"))
 (segment (start 62 65.6375) (end 62 65.990552) (width 0.2) (layer "F.Cu") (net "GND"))
 (segment (start 67.325 63.325) (end 67 63) (width 0.2) (layer "F.Cu") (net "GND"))
 (via (at 70 56) (size 0.6) (drill 0.3) (layers "F.Cu" "B.Cu") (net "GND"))
 (via (at 62 56) (size 0.6) (drill 0.3) (layers "F.Cu" "B.Cu") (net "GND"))
 (via (at 51.5 65.5) (size 0.6) (drill 0.3) (layers "F.Cu" "B.Cu") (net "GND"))
 (via (at 50.5 53) (size 0.6) (drill 0.3) (layers "F.Cu" "B.Cu") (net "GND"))
 (via (at 67 63) (size 0.6) (drill 0.3) (layers "F.Cu" "B.Cu") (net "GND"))
 (segment (start 50.5 53) (end 52 54.5) (width 0.2) (layer "B.Cu") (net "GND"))
 (segment (start 62 56) (end 70 56) (width 0.2) (layer "B.Cu") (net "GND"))
 (segment (start 51.5 62.54) (end 51.5 65.5) (width 0.2) (layer "B.Cu") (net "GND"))
 (segment (start 48.5 59.54) (end 51.5 62.54) (width 0.2) (layer "B.Cu") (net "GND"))
 (segment (start 52 54.5) (end 69.5 54.5) (width 0.2) (layer "B.Cu") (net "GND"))
 (segment (start 50.5 57.54) (end 50.5 53) (width 0.2) (layer "B.Cu") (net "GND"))
 (segment (start 67 63) (end 67 59) (width 0.2) (layer "B.Cu") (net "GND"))
 (segment (start 67 59) (end 70 56) (width 0.2) (layer "B.Cu") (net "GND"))
 (segment (start 48.5 59.54) (end 50.5 57.54) (width 0.2) (layer "B.Cu") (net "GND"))
 (segment (start 59 57.5) (end 61.05 55.45) (width 0.2) (layer "F.Cu") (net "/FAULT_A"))
 (segment (start 61.05 55.45) (end 61.05 54.6375) (width 0.2) (layer "F.Cu") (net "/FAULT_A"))
 (segment (start 65.5875 52.5) (end 65.0875 52.5) (width 0.2) (layer "F.Cu") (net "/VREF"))
 (segment (start 63.3125 66) (end 62.95 65.6375) (width 0.2) (layer "F.Cu") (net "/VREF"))
 (segment (start 65.0875 52.5) (end 62.95 54.6375) (width 0.2) (layer "F.Cu") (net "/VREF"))
 (segment (start 63 59.5) (end 63 59) (width 0.2) (layer "F.Cu") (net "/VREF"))
 (segment (start 65.5 62) (end 65.5 65.5) (width 0.2) (layer "F.Cu") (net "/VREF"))
 (segment (start 65 66) (end 63.3125 66) (width 0.2) (layer "F.Cu") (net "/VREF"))
 (segment (start 65.5 65.5) (end 65 66) (width 0.2) (layer "F.Cu") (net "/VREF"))
 (segment (start 63 59) (end 62.95 58.95) (width 0.2) (layer "F.Cu") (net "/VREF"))
 (segment (start 62.95 58.95) (end 62.95 54.6375) (width 0.2) (layer "F.Cu") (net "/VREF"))
 (segment (start 63 59.5) (end 65.5 62) (width 0.2) (layer "F.Cu") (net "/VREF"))
 (segment (start 50.5 62.5875) (end 50.5 66.5) (width 0.2) (layer "F.Cu") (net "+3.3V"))
 (segment (start 50.5 66.5) (end 56 66.5) (width 0.2) (layer "F.Cu") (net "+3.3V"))
 (segment (start 69.45 52.5) (end 69.5 52.55) (width 0.2) (layer "F.Cu") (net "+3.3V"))
 (segment (start 56.5 62.5) (end 60.1875 62.5) (width 0.2) (layer "F.Cu") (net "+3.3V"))
 (segment (start 48.5 57) (end 52.0875 57) (width 0.2) (layer "F.Cu") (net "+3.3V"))
 (segment (start 71 67) (end 71 64.05) (width 0.2) (layer "F.Cu") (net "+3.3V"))
 (segment (start 69.5 62.55) (end 71 61.05) (width 0.2) (layer "F.Cu") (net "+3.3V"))
 (segment (start 55.4125 58) (end 61.05 52.3625) (width 0.2) (layer "F.Cu") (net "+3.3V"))
 (segment (start 56.5 67) (end 71 67) (width 0.2) (layer "F.Cu") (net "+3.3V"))
 (segment (start 52.0875 61) (end 52.0875 57) (width 0.2) (layer "F.Cu") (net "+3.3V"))
 (segment (start 56 66.5) (end 56.5 66) (width 0.2) (layer "F.Cu") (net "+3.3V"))
 (segment (start 60.1875 62.5) (end 61.05 63.3625) (width 0.2) (layer "F.Cu") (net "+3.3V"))
 (segment (start 71 52.5) (end 70.95 52.55) (width 0.2) (layer "F.Cu") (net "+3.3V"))
 (segment (start 71 61.05) (end 71 52.5) (width 0.2) (layer "F.Cu") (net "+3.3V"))
 (segment (start 67.4125 52.5) (end 69.45 52.5) (width 0.2) (layer "F.Cu") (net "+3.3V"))
 (segment (start 53.0875 58) (end 55.4125 58) (width 0.2) (layer "F.Cu") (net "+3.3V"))
 (segment (start 52.0875 57) (end 53.0875 58) (width 0.2) (layer "F.Cu") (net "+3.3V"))
 (segment (start 70.95 52.55) (end 69.5 52.55) (width 0.2) (layer "F.Cu") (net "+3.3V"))
 (segment (start 56 66.5) (end 56.5 67) (width 0.2) (layer "F.Cu") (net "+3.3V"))
 (segment (start 52.0875 61) (end 50.5 62.5875) (width 0.2) (layer "F.Cu") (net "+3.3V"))
 (segment (start 56.5 66) (end 56.5 62.5) (width 0.2) (layer "F.Cu") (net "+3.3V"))
 (segment (start 71 64.05) (end 69.5 62.55) (width 0.2) (layer "F.Cu") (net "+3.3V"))
 (segment (start 57 61) (end 60.5875 61) (width 0.2) (layer "F.Cu") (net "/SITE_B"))
 (segment (start 53.9125 61) (end 53.9125 64) (width 0.2) (layer "F.Cu") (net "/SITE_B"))
 (segment (start 57 59.5) (end 57 61) (width 0.2) (layer "F.Cu") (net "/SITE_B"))
 (segment (start 60.5875 61) (end 62.95 63.3625) (width 0.2) (layer "F.Cu") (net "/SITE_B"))
 (segment (start 56.5 61) (end 57 61) (width 0.2) (layer "F.Cu") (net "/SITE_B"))
 (segment (start 56.5 61) (end 53.9125 61) (width 0.2) (layer "F.Cu") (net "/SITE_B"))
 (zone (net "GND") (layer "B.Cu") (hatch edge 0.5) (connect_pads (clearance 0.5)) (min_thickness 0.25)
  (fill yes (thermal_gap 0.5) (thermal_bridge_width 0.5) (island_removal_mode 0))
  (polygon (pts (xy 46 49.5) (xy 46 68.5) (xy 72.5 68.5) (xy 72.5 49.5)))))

